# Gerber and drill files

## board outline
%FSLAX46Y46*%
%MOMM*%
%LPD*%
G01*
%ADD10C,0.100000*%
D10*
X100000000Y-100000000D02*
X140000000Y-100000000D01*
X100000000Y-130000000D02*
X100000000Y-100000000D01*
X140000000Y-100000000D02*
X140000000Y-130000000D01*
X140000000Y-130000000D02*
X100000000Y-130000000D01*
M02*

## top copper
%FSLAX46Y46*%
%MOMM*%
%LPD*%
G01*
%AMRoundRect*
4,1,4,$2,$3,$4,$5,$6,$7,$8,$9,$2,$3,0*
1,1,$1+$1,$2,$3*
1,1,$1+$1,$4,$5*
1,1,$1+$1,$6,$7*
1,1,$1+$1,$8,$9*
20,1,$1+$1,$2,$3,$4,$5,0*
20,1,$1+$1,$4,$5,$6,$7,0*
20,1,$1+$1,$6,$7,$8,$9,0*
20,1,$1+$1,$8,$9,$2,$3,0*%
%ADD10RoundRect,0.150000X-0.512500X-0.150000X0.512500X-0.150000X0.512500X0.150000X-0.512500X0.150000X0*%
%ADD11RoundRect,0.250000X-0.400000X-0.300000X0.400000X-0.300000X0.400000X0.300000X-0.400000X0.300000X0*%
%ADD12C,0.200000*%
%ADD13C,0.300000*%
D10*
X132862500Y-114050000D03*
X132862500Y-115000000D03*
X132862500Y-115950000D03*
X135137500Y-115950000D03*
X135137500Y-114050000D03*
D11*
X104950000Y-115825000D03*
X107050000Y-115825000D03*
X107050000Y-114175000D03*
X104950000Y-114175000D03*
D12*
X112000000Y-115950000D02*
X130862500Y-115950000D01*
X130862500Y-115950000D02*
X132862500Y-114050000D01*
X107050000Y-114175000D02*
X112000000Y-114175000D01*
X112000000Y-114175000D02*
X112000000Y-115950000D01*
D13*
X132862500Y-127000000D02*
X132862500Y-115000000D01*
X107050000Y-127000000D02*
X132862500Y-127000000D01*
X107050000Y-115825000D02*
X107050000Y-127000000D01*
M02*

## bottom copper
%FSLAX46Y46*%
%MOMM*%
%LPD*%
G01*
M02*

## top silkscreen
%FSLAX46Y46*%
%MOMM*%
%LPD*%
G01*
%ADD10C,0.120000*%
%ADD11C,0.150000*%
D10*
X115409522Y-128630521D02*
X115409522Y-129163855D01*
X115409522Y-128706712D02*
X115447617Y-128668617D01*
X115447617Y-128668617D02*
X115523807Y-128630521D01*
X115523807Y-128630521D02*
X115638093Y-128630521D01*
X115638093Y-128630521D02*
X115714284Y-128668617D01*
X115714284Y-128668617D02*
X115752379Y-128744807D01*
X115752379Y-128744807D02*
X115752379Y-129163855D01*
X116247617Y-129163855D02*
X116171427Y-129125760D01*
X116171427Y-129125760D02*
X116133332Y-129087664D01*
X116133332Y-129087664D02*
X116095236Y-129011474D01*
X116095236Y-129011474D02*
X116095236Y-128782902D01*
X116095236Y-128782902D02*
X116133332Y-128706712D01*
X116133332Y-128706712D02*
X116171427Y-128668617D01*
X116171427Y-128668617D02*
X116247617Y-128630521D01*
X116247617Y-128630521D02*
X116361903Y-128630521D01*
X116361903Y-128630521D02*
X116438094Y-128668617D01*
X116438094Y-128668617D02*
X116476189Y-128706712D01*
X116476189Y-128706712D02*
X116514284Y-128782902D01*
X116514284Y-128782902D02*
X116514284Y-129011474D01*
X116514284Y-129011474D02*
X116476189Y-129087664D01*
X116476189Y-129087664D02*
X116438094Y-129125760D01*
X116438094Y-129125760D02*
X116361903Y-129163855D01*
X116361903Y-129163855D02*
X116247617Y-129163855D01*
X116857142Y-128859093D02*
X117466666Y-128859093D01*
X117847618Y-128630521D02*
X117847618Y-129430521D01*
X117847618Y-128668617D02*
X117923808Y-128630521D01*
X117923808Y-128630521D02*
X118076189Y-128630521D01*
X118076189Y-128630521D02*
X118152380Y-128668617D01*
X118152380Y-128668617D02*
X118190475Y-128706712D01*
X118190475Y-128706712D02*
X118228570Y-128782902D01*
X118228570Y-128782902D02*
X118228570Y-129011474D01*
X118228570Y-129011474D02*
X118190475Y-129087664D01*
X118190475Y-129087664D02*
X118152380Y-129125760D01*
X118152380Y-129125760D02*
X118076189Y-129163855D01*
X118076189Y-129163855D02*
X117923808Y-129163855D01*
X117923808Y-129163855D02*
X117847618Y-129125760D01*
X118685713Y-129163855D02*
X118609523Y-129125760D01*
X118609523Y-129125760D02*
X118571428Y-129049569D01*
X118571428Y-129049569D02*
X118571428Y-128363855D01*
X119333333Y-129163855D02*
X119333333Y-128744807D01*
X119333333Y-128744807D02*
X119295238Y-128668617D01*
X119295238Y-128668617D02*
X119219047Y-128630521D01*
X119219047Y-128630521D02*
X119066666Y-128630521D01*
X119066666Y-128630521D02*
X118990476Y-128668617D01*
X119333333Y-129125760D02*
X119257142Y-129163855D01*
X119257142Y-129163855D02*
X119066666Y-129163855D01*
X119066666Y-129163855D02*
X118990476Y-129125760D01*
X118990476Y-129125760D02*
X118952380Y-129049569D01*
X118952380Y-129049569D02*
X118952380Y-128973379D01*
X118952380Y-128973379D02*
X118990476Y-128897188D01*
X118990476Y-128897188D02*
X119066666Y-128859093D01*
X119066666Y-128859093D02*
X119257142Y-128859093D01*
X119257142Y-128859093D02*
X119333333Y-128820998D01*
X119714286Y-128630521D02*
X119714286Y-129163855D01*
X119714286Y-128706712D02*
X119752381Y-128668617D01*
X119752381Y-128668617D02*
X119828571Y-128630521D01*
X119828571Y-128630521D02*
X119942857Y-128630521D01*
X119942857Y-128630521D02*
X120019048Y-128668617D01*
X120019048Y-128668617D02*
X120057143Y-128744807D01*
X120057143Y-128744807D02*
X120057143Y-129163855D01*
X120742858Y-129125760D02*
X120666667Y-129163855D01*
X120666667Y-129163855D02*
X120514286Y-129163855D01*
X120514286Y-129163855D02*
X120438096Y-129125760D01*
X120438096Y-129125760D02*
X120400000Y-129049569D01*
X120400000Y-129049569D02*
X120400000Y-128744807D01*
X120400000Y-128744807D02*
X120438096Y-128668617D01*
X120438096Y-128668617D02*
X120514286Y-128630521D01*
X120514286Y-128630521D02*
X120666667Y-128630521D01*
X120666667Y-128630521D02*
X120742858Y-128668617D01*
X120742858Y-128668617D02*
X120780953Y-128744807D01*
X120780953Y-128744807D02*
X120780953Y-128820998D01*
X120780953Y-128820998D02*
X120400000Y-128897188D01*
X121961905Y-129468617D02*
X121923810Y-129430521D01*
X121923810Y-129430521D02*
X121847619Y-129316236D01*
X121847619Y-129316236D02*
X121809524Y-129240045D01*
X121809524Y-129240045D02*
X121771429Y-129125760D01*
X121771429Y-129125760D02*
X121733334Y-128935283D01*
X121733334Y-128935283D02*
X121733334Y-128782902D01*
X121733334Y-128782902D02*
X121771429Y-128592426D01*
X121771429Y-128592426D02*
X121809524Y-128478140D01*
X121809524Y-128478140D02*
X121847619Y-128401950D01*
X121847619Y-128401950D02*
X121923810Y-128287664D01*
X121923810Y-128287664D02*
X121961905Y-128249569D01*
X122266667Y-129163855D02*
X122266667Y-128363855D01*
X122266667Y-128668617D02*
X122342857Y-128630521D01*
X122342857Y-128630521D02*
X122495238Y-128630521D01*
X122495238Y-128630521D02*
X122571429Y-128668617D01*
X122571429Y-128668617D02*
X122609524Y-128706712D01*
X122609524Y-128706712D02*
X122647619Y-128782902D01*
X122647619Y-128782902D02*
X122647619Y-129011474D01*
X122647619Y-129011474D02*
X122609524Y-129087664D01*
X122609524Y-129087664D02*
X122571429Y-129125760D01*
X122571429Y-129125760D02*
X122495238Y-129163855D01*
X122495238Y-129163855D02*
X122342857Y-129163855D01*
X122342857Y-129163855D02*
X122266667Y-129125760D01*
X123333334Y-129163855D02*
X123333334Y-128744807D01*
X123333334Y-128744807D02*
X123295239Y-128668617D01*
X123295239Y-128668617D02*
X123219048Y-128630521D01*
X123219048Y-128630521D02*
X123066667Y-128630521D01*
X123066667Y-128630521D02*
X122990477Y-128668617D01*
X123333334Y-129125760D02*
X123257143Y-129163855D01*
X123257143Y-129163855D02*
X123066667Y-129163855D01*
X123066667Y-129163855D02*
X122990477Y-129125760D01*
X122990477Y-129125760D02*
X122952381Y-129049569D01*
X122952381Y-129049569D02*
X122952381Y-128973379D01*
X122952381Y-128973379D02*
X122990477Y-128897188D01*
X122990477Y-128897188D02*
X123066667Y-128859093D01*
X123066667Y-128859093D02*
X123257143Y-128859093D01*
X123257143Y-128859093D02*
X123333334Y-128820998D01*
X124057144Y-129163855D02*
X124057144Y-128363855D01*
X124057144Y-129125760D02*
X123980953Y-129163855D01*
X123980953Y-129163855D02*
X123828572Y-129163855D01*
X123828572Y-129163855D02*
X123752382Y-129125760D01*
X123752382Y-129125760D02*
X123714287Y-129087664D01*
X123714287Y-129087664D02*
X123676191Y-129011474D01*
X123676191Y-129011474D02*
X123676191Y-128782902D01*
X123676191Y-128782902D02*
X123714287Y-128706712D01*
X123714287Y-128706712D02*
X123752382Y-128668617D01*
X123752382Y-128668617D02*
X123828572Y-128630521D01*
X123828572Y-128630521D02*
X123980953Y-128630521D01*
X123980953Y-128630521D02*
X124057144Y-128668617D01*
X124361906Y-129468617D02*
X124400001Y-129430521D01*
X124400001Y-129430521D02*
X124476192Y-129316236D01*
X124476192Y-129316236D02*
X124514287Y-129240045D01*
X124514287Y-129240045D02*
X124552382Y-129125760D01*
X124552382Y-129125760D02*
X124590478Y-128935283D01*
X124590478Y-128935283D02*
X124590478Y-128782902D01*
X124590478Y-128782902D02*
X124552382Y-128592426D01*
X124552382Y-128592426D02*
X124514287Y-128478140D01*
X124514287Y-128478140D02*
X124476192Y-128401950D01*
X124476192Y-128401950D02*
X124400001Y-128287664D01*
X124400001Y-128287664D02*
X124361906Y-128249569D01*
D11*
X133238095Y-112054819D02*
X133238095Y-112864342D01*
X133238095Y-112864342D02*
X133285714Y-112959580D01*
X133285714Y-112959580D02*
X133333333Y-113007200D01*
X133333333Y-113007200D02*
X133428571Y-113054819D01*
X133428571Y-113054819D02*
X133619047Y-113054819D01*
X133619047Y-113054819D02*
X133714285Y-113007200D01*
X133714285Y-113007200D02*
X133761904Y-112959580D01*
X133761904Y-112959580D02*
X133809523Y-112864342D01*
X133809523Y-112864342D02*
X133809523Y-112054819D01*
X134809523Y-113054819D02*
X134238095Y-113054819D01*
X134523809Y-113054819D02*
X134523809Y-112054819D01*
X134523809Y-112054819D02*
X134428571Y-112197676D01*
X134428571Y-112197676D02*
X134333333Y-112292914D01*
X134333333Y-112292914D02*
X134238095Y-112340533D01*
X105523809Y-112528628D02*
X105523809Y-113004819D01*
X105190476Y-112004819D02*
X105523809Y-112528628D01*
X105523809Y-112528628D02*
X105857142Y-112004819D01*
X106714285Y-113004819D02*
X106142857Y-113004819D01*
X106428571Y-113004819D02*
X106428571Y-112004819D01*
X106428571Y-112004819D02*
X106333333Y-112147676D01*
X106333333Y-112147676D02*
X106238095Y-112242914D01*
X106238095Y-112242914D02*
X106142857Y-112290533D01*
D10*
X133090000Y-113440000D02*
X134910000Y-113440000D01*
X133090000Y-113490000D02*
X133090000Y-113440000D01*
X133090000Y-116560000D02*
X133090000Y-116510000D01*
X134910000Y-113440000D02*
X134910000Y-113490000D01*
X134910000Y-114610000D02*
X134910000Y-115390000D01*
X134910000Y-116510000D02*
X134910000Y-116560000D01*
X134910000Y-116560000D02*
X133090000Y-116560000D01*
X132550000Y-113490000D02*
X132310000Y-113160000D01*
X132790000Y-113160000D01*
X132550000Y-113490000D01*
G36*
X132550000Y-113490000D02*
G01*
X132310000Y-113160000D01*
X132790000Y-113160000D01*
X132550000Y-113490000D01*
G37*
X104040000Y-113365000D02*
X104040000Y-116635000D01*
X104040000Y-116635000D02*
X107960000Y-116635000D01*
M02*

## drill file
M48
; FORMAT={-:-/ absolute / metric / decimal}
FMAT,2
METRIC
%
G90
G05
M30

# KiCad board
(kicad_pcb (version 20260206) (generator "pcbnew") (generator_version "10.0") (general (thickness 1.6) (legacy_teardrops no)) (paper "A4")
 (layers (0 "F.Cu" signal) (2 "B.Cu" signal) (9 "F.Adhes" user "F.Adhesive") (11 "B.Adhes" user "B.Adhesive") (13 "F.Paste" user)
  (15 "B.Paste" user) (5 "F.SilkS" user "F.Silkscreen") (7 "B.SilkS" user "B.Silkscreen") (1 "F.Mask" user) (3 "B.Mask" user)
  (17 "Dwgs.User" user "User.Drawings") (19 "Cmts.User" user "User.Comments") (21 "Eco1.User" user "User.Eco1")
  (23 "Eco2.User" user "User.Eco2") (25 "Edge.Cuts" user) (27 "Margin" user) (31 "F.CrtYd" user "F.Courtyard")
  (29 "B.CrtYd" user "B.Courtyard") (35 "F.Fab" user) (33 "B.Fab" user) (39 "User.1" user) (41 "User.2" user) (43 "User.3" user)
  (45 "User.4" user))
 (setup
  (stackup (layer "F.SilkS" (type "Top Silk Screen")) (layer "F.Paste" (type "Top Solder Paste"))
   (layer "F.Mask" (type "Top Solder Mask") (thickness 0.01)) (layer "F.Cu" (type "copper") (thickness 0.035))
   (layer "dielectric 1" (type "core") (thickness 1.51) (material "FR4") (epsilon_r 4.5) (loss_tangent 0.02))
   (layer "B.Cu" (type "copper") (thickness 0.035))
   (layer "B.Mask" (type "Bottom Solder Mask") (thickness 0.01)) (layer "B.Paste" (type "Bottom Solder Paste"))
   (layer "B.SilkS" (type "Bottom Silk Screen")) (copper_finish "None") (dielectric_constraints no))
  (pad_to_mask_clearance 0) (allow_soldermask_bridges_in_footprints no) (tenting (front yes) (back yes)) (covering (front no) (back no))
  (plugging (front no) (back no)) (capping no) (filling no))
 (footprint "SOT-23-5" (layer "F.Cu") (at 134 115)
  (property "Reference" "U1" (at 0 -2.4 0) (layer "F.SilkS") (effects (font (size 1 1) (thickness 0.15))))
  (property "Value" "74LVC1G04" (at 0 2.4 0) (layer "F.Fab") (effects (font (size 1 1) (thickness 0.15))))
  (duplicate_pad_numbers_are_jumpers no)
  (fp_line (start -0.91 -1.56) (end 0.91 -1.56) (stroke (width 0.12) (type solid)) (layer "F.SilkS"))
  (fp_line (start -0.91 -1.51) (end -0.91 -1.56) (stroke (width 0.12) (type solid)) (layer "F.SilkS"))
  (fp_line (start -0.91 1.56) (end -0.91 1.51) (stroke (width 0.12) (type solid)) (layer "F.SilkS"))
  (fp_line (start 0.91 -1.56) (end 0.91 -1.51) (stroke (width 0.12) (type solid)) (layer "F.SilkS"))
  (fp_line (start 0.91 -0.39) (end 0.91 0.39) (stroke (width 0.12) (type solid)) (layer "F.SilkS"))
  (fp_line (start 0.91 1.51) (end 0.91 1.56) (stroke (width 0.12) (type solid)) (layer "F.SilkS"))
  (fp_line (start 0.91 1.56) (end -0.91 1.56) (stroke (width 0.12) (type solid)) (layer "F.SilkS"))
  (fp_poly (pts (xy -1.45 -1.51) (xy -1.69 -1.84) (xy -1.21 -1.84)) (stroke (width 0.12) (type solid)) (fill yes) (layer "F.SilkS"))
  (pad "1" smd roundrect (at -1.1375 -0.95) (size 1.325 0.6) (layers "F.Cu" "F.Mask" "F.Paste") (roundrect_rratio 0.25) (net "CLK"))
  (pad "2" smd roundrect (at -1.1375 0) (size 1.325 0.6) (layers "F.Cu" "F.Mask" "F.Paste") (roundrect_rratio 0.25) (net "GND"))
  (pad "3" smd roundrect (at -1.1375 0.95) (size 1.325 0.6) (layers "F.Cu" "F.Mask" "F.Paste") (roundrect_rratio 0.25))
  (pad "4" smd roundrect (at 1.1375 0.95) (size 1.325 0.6) (layers "F.Cu" "F.Mask" "F.Paste") (roundrect_rratio 0.25))
  (pad "5" smd roundrect (at 1.1375 -0.95) (size 1.325 0.6) (layers "F.Cu" "F.Mask" "F.Paste") (roundrect_rratio 0.25) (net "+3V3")))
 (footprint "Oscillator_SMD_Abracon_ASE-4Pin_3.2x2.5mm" (layer "F.Cu") (at 106 115)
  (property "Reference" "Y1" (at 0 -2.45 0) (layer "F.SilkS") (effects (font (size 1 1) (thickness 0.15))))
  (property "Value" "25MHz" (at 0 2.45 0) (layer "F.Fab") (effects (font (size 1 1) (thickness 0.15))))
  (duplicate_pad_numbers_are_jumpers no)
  (fp_line (start -1.96 -1.635) (end -1.96 1.635) (stroke (width 0.12) (type solid)) (layer "F.SilkS"))
  (fp_line (start -1.96 1.635) (end 1.96 1.635) (stroke (width 0.12) (type solid)) (layer "F.SilkS"))
  (pad "1" smd roundrect (at -1.05 0.825) (size 1.3 1.1) (layers "F.Cu" "F.Mask" "F.Paste") (roundrect_rratio 0.227273) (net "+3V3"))
  (pad "2" smd roundrect (at 1.05 0.825) (size 1.3 1.1) (layers "F.Cu" "F.Mask" "F.Paste") (roundrect_rratio 0.227273) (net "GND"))
  (pad "3" smd roundrect (at 1.05 -0.825) (size 1.3 1.1) (layers "F.Cu" "F.Mask" "F.Paste") (roundrect_rratio 0.227273) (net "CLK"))
  (pad "4" smd roundrect (at -1.05 -0.825) (size 1.3 1.1) (layers "F.Cu" "F.Mask" "F.Paste") (roundrect_rratio 0.227273) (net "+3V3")))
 (gr_line (start 100 100) (end 140 100) (stroke (width 0.1) (type default)) (layer "Edge.Cuts"))
 (gr_line (start 100 130) (end 100 100) (stroke (width 0.1) (type default)) (layer "Edge.Cuts"))
 (gr_line (start 140 100) (end 140 130) (stroke (width 0.1) (type default)) (layer "Edge.Cuts"))
 (gr_line (start 140 130) (end 100 130) (stroke (width 0.1) (type default)) (layer "Edge.Cuts"))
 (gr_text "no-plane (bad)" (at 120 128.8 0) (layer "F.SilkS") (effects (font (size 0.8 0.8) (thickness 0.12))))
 (segment (start 112 115.95) (end 130.8625 115.95) (width 0.2) (layer "F.Cu") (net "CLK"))
 (segment (start 130.8625 115.95) (end 132.8625 114.05) (width 0.2) (layer "F.Cu") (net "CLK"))
 (segment (start 107.05 114.175) (end 112 114.175) (width 0.2) (layer "F.Cu") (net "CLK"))
 (segment (start 112 114.175) (end 112 115.95) (width 0.2) (layer "F.Cu") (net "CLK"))
 (segment (start 132.8625 127) (end 132.8625 115) (width 0.3) (layer "F.Cu") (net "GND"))
 (segment (start 107.05 127) (end 132.8625 127) (width 0.3) (layer "F.Cu") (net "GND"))
 (segment (start 107.05 115.825) (end 107.05 127) (width 0.3) (layer "F.Cu") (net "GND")))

